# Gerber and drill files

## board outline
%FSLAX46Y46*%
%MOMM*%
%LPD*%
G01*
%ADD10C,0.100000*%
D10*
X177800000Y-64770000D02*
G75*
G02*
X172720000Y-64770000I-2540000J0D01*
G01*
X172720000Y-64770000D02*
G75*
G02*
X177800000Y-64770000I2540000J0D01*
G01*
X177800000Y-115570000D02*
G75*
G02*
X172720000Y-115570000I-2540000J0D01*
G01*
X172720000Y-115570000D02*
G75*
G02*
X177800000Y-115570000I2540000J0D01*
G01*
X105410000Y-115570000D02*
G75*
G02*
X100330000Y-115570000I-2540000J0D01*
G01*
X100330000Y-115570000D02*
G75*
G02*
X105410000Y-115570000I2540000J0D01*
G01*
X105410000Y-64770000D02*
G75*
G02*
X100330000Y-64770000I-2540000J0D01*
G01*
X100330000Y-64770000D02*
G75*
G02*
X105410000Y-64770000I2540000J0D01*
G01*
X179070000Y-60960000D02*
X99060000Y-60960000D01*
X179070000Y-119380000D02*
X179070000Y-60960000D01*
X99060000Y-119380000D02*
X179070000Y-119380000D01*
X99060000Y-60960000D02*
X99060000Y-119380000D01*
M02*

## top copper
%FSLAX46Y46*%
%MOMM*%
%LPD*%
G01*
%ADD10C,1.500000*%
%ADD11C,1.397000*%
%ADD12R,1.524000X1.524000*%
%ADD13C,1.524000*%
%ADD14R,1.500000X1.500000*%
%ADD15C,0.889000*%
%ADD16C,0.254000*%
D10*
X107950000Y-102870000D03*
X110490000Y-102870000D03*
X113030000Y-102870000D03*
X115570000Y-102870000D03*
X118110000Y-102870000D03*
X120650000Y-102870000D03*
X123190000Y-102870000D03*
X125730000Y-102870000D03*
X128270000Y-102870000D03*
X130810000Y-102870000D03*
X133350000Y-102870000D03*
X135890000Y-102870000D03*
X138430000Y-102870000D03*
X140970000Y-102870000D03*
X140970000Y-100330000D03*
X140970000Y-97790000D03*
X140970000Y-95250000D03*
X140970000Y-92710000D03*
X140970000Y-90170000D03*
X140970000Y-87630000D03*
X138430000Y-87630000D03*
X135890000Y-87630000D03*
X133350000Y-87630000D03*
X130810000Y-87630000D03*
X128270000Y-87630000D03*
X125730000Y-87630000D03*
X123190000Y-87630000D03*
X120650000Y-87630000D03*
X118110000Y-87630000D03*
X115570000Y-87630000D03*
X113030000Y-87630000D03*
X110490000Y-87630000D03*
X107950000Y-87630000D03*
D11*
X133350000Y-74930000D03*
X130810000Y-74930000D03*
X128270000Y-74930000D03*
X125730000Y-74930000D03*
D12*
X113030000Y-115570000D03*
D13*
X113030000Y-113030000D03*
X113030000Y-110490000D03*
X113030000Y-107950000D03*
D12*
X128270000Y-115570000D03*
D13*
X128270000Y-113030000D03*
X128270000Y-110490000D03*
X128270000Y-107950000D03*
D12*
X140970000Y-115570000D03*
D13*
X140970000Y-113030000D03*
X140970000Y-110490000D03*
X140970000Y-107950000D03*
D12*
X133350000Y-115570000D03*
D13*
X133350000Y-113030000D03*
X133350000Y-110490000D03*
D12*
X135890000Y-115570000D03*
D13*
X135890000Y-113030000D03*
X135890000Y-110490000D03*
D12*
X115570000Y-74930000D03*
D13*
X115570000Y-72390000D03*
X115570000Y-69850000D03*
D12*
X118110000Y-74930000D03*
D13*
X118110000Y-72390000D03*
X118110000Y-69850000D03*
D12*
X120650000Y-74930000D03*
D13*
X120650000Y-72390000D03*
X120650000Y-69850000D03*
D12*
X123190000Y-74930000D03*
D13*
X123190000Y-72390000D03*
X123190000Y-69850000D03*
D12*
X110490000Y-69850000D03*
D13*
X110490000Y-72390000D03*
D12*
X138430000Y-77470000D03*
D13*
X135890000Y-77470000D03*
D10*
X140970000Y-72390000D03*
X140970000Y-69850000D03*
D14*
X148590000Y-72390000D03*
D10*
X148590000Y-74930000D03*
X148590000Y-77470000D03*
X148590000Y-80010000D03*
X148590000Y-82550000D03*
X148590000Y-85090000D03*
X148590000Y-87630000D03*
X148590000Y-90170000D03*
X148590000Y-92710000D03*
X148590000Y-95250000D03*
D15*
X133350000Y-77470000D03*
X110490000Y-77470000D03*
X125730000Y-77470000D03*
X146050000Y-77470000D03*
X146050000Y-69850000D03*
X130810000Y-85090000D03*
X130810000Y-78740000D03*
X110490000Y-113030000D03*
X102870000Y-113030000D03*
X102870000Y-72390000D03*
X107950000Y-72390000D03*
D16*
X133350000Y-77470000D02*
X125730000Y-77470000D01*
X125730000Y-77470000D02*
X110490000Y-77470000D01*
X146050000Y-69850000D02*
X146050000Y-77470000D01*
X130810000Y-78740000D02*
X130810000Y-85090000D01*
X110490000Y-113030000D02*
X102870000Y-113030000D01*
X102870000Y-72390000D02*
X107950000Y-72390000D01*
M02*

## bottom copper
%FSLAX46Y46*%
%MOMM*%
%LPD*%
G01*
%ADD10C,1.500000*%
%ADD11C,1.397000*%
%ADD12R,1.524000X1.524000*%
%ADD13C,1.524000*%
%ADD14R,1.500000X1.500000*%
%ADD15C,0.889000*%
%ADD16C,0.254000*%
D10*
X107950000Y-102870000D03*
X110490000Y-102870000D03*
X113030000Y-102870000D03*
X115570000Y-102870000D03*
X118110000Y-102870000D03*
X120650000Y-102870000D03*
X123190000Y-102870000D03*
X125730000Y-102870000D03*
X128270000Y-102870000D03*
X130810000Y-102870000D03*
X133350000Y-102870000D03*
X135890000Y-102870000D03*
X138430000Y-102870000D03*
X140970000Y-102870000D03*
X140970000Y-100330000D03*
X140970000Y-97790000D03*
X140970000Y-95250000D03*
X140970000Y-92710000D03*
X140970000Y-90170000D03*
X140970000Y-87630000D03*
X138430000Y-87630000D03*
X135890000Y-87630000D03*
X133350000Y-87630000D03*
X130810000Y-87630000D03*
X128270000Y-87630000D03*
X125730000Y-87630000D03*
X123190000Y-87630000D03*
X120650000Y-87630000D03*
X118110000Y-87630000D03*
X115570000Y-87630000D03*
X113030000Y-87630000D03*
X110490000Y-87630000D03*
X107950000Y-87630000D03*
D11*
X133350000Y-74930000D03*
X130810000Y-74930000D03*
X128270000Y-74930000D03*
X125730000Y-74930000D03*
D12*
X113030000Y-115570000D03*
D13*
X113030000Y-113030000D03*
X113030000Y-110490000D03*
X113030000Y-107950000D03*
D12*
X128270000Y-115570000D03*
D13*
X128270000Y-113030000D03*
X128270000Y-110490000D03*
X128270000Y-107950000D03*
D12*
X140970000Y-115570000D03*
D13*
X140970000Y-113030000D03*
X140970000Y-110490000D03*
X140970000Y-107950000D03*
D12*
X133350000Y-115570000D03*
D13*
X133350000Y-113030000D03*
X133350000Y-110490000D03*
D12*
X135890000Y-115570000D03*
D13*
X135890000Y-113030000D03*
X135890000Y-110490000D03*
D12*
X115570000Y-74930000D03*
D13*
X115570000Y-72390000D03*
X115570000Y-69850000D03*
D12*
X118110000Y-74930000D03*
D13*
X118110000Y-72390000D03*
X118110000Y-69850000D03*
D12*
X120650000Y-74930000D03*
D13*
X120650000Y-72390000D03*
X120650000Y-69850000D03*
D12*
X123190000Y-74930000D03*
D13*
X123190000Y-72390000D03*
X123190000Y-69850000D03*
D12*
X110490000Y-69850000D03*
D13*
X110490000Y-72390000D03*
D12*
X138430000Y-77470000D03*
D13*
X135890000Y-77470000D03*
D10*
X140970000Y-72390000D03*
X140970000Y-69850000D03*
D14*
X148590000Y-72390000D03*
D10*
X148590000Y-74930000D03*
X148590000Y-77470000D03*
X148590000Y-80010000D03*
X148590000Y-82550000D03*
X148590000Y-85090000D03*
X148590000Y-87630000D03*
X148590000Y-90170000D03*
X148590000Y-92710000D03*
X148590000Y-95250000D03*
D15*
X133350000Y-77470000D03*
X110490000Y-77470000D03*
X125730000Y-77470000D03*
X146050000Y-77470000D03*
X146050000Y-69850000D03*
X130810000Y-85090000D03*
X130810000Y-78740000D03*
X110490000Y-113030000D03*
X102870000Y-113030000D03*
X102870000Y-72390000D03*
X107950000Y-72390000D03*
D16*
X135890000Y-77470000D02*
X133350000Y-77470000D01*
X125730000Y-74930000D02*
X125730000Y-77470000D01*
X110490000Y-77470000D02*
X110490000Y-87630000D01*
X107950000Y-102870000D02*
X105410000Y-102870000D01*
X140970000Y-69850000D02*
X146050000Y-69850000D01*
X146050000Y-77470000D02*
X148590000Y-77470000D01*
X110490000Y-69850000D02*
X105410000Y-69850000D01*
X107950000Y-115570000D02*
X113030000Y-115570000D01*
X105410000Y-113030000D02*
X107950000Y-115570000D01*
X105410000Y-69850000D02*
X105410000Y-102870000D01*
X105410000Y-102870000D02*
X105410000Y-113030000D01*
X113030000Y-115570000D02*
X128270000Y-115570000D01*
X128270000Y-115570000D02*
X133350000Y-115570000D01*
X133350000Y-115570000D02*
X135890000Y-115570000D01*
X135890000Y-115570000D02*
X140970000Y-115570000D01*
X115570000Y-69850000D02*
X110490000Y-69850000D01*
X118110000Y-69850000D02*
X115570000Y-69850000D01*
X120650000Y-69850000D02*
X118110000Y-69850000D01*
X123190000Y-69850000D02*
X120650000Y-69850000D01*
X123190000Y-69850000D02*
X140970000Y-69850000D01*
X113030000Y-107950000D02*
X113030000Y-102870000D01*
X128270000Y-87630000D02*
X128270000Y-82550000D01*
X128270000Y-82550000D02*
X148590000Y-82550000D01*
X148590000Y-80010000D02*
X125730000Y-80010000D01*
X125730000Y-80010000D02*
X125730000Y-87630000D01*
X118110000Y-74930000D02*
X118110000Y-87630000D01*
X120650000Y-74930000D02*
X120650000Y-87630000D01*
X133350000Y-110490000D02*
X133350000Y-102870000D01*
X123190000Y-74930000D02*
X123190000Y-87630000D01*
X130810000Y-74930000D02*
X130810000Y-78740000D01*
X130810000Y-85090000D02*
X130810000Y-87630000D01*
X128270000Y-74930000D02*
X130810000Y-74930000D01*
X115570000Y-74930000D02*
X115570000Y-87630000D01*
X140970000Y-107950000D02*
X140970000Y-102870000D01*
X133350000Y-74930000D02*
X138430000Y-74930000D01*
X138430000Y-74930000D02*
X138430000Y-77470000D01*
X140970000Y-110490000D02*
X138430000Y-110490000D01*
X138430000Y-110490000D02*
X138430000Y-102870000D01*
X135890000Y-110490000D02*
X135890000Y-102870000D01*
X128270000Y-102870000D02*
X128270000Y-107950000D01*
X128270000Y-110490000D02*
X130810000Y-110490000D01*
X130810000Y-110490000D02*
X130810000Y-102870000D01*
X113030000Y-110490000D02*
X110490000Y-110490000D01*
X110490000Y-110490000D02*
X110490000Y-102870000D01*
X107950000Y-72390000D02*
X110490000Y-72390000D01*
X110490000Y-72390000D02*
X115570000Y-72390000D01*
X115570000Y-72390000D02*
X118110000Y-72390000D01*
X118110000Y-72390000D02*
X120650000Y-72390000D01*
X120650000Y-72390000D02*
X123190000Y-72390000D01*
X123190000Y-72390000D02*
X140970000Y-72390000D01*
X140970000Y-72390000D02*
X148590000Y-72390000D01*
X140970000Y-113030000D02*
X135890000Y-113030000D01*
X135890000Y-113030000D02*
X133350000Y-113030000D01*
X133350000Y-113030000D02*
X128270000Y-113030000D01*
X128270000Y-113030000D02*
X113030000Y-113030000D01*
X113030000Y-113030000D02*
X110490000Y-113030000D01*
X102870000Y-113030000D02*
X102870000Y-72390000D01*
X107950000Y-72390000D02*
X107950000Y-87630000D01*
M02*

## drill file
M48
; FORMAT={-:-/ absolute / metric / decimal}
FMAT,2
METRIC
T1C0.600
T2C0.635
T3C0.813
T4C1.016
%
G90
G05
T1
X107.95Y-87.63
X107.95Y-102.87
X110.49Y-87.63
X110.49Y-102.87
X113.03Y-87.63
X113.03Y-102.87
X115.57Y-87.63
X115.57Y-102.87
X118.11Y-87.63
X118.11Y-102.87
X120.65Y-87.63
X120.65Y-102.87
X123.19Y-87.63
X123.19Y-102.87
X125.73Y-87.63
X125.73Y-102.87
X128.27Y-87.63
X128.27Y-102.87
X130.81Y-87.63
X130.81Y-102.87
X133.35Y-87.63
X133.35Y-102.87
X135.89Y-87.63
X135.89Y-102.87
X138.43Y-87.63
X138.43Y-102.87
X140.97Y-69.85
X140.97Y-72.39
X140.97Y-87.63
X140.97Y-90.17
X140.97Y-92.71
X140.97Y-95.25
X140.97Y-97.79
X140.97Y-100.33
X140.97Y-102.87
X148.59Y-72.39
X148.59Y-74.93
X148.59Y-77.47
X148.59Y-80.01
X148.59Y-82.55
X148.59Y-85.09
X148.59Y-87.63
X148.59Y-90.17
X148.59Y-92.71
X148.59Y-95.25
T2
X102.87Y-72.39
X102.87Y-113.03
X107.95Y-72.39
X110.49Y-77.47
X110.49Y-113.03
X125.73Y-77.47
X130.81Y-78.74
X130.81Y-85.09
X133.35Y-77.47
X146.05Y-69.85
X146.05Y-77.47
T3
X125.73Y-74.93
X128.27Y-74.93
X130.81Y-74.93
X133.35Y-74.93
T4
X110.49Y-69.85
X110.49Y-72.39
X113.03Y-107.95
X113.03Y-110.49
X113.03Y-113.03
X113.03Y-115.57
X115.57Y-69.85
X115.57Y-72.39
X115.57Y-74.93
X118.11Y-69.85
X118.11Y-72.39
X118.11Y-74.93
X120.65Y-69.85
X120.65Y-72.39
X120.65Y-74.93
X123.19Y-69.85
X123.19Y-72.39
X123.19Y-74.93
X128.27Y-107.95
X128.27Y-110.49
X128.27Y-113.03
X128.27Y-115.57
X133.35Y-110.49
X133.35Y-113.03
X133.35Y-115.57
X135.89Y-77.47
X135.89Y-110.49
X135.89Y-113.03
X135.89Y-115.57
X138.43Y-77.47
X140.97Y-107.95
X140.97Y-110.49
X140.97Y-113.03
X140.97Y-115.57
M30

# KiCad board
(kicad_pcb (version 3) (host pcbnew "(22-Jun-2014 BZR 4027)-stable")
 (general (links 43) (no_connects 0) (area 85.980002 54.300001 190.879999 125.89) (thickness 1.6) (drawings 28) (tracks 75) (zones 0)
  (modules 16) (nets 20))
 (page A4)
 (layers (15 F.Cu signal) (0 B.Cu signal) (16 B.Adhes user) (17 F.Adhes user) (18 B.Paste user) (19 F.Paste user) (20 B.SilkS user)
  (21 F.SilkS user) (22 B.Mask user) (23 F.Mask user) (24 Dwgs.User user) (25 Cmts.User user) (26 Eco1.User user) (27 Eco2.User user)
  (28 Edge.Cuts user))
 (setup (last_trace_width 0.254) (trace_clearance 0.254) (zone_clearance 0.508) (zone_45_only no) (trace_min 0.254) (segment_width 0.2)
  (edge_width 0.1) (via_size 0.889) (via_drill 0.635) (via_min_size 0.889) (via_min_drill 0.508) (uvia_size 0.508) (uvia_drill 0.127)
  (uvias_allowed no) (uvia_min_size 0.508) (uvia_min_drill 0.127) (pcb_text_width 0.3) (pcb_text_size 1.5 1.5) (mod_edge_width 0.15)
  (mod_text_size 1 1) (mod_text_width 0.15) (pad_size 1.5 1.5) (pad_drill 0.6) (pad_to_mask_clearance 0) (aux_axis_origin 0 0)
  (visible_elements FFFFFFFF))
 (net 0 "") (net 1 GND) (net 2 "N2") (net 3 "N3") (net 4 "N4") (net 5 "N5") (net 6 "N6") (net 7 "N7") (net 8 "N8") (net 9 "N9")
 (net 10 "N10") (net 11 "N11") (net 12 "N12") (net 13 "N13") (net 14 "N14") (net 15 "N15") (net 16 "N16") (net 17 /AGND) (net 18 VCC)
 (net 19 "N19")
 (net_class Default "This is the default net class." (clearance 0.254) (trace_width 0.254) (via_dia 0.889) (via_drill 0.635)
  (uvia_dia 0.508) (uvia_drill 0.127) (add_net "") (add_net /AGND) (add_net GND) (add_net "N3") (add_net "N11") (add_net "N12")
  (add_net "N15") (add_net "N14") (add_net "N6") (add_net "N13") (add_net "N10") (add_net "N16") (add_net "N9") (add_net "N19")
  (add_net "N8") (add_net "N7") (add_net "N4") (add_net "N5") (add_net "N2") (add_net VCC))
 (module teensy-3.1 (layer F.Cu) (at 124.46 95.25 90)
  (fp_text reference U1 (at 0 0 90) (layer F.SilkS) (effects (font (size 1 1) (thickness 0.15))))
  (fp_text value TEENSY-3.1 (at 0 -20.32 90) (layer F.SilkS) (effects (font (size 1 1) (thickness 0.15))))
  (pad 1 thru_hole circle (at -7.62 -16.51 90) (size 1.5 1.5) (drill 0.6) (layers *.Cu *.Mask F.SilkS) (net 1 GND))
  (pad 2 thru_hole circle (at -7.62 -13.97 90) (size 1.5 1.5) (drill 0.6) (layers *.Cu *.Mask F.SilkS) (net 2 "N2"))
  (pad 3 thru_hole circle (at -7.62 -11.43 90) (size 1.5 1.5) (drill 0.6) (layers *.Cu *.Mask F.SilkS) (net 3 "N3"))
  (pad 4 thru_hole circle (at -7.62 -8.89 90) (size 1.5 1.5) (drill 0.6) (layers *.Cu *.Mask F.SilkS))
  (pad 5 thru_hole circle (at -7.62 -6.35 90) (size 1.5 1.5) (drill 0.6) (layers *.Cu *.Mask F.SilkS))
  (pad 6 thru_hole circle (at -7.62 -3.81 90) (size 1.5 1.5) (drill 0.6) (layers *.Cu *.Mask F.SilkS))
  (pad 7 thru_hole circle (at -7.62 -1.27 90) (size 1.5 1.5) (drill 0.6) (layers *.Cu *.Mask F.SilkS))
  (pad 8 thru_hole circle (at -7.62 1.27 90) (size 1.5 1.5) (drill 0.6) (layers *.Cu *.Mask F.SilkS))
  (pad 9 thru_hole circle (at -7.62 3.81 90) (size 1.5 1.5) (drill 0.6) (layers *.Cu *.Mask F.SilkS) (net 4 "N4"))
  (pad 10 thru_hole circle (at -7.62 6.35 90) (size 1.5 1.5) (drill 0.6) (layers *.Cu *.Mask F.SilkS) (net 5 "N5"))
  (pad 11 thru_hole circle (at -7.62 8.89 90) (size 1.5 1.5) (drill 0.6) (layers *.Cu *.Mask F.SilkS) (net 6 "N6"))
  (pad 12 thru_hole circle (at -7.62 11.43 90) (size 1.5 1.5) (drill 0.6) (layers *.Cu *.Mask F.SilkS) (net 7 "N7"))
  (pad 13 thru_hole circle (at -7.62 13.97 90) (size 1.5 1.5) (drill 0.6) (layers *.Cu *.Mask F.SilkS) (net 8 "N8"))
  (pad 14 thru_hole circle (at -7.62 16.51 90) (size 1.5 1.5) (drill 0.6) (layers *.Cu *.Mask F.SilkS) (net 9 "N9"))
  (pad 15 thru_hole circle (at -5.08 16.51 90) (size 1.5 1.5) (drill 0.6) (layers *.Cu *.Mask F.SilkS))
  (pad 16 thru_hole circle (at -2.54 16.51 90) (size 1.5 1.5) (drill 0.6) (layers *.Cu *.Mask F.SilkS))
  (pad 17 thru_hole circle (at 0 16.51 90) (size 1.5 1.5) (drill 0.6) (layers *.Cu *.Mask F.SilkS))
  (pad 18 thru_hole circle (at 2.54 16.51 90) (size 1.5 1.5) (drill 0.6) (layers *.Cu *.Mask F.SilkS))
  (pad 19 thru_hole circle (at 5.08 16.51 90) (size 1.5 1.5) (drill 0.6) (layers *.Cu *.Mask F.SilkS))
  (pad 20 thru_hole circle (at 7.62 16.51 90) (size 1.5 1.5) (drill 0.6) (layers *.Cu *.Mask F.SilkS))
  (pad 21 thru_hole circle (at 7.62 13.97 90) (size 1.5 1.5) (drill 0.6) (layers *.Cu *.Mask F.SilkS))
  (pad 22 thru_hole circle (at 7.62 11.43 90) (size 1.5 1.5) (drill 0.6) (layers *.Cu *.Mask F.SilkS))
  (pad 23 thru_hole circle (at 7.62 8.89 90) (size 1.5 1.5) (drill 0.6) (layers *.Cu *.Mask F.SilkS))
  (pad 24 thru_hole circle (at 7.62 6.35 90) (size 1.5 1.5) (drill 0.6) (layers *.Cu *.Mask F.SilkS) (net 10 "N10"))
  (pad 25 thru_hole circle (at 7.62 3.81 90) (size 1.5 1.5) (drill 0.6) (layers *.Cu *.Mask F.SilkS) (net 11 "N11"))
  (pad 26 thru_hole circle (at 7.62 1.27 90) (size 1.5 1.5) (drill 0.6) (layers *.Cu *.Mask F.SilkS) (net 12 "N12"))
  (pad 27 thru_hole circle (at 7.62 -1.27 90) (size 1.5 1.5) (drill 0.6) (layers *.Cu *.Mask F.SilkS) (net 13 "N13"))
  (pad 28 thru_hole circle (at 7.62 -3.81 90) (size 1.5 1.5) (drill 0.6) (layers *.Cu *.Mask F.SilkS) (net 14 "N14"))
  (pad 29 thru_hole circle (at 7.62 -6.35 90) (size 1.5 1.5) (drill 0.6) (layers *.Cu *.Mask F.SilkS) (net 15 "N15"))
  (pad 30 thru_hole circle (at 7.62 -8.89 90) (size 1.5 1.5) (drill 0.6) (layers *.Cu *.Mask F.SilkS) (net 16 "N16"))
  (pad 31 thru_hole circle (at 7.62 -11.43 90) (size 1.5 1.5) (drill 0.6) (layers *.Cu *.Mask F.SilkS))
  (pad 32 thru_hole circle (at 7.62 -13.97 90) (size 1.5 1.5) (drill 0.6) (layers *.Cu *.Mask F.SilkS) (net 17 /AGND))
  (pad 33 thru_hole circle (at 7.62 -16.51 90) (size 1.5 1.5) (drill 0.6) (layers *.Cu *.Mask F.SilkS) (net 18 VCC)))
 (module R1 (layer F.Cu) (at 132.08 74.93 180) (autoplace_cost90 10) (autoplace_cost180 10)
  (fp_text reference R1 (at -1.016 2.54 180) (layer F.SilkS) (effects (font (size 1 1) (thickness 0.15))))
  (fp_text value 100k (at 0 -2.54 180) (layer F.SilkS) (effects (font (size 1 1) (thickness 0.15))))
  (pad 1 thru_hole circle (at -1.27 0 180) (size 1.397 1.397) (drill 0.8128) (layers *.Cu *.Mask F.SilkS) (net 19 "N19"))
  (pad 2 thru_hole circle (at 1.27 0 180) (size 1.397 1.397) (drill 0.8128) (layers *.Cu *.Mask F.SilkS) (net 10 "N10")))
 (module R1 (layer F.Cu) (at 127 74.93 180) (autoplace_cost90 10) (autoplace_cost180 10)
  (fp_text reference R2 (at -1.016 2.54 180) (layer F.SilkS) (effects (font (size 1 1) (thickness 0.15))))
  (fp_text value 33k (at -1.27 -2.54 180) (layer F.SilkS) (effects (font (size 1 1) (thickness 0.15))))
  (pad 1 thru_hole circle (at -1.27 0 180) (size 1.397 1.397) (drill 0.8128) (layers *.Cu *.Mask F.SilkS) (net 10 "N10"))
  (pad 2 thru_hole circle (at 1.27 0 180) (size 1.397 1.397) (drill 0.8128) (layers *.Cu *.Mask F.SilkS) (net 17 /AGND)))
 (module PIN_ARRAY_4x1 (layer F.Cu) (at 113.03 111.76 90)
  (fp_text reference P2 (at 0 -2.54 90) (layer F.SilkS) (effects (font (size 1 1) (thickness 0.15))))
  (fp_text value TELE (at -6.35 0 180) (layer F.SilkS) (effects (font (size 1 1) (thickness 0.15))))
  (pad 1 thru_hole rect (at -3.81 0 90) (size 1.524 1.524) (drill 1.016) (layers *.Cu *.Mask F.SilkS) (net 1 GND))
  (pad 2 thru_hole circle (at -1.27 0 90) (size 1.524 1.524) (drill 1.016) (layers *.Cu *.Mask F.SilkS) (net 18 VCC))
  (pad 3 thru_hole circle (at 1.27 0 90) (size 1.524 1.524) (drill 1.016) (layers *.Cu *.Mask F.SilkS) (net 2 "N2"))
  (pad 4 thru_hole circle (at 3.81 0 90) (size 1.524 1.524) (drill 1.016) (layers *.Cu *.Mask F.SilkS) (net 3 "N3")))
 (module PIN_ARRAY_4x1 (layer F.Cu) (at 128.27 111.76 90)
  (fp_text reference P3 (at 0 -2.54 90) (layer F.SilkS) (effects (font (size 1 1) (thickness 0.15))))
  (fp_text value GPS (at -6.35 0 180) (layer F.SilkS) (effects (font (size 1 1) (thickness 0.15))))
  (pad 1 thru_hole rect (at -3.81 0 90) (size 1.524 1.524) (drill 1.016) (layers *.Cu *.Mask F.SilkS) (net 1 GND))
  (pad 2 thru_hole circle (at -1.27 0 90) (size 1.524 1.524) (drill 1.016) (layers *.Cu *.Mask F.SilkS) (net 18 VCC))
  (pad 3 thru_hole circle (at 1.27 0 90) (size 1.524 1.524) (drill 1.016) (layers *.Cu *.Mask F.SilkS) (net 5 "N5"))
  (pad 4 thru_hole circle (at 3.81 0 90) (size 1.524 1.524) (drill 1.016) (layers *.Cu *.Mask F.SilkS) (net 4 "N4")))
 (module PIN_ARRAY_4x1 (layer F.Cu) (at 140.97 111.76 90)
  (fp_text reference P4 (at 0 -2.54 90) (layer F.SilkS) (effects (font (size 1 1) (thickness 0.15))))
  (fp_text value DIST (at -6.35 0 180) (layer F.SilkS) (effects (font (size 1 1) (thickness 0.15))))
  (pad 1 thru_hole rect (at -3.81 0 90) (size 1.524 1.524) (drill 1.016) (layers *.Cu *.Mask F.SilkS) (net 1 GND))
  (pad 2 thru_hole circle (at -1.27 0 90) (size 1.524 1.524) (drill 1.016) (layers *.Cu *.Mask F.SilkS) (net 18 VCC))
  (pad 3 thru_hole circle (at 1.27 0 90) (size 1.524 1.524) (drill 1.016) (layers *.Cu *.Mask F.SilkS) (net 8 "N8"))
  (pad 4 thru_hole circle (at 3.81 0 90) (size 1.524 1.524) (drill 1.016) (layers *.Cu *.Mask F.SilkS) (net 9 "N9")))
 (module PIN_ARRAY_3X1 (layer F.Cu) (at 133.35 113.03 90)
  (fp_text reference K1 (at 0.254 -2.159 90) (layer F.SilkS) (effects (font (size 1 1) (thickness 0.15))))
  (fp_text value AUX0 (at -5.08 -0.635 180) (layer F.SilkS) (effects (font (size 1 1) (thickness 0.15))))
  (pad 1 thru_hole rect (at -2.54 0 90) (size 1.524 1.524) (drill 1.016) (layers *.Cu *.Mask F.SilkS) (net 1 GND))
  (pad 2 thru_hole circle (at 0 0 90) (size 1.524 1.524) (drill 1.016) (layers *.Cu *.Mask F.SilkS) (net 18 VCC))
  (pad 3 thru_hole circle (at 2.54 0 90) (size 1.524 1.524) (drill 1.016) (layers *.Cu *.Mask F.SilkS) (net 6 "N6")))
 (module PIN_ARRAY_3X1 (layer F.Cu) (at 135.89 113.03 90)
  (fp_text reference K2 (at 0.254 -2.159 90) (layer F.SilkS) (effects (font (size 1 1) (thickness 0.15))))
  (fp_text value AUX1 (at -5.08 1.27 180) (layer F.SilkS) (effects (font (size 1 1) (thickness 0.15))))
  (pad 1 thru_hole rect (at -2.54 0 90) (size 1.524 1.524) (drill 1.016) (layers *.Cu *.Mask F.SilkS) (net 1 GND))
  (pad 2 thru_hole circle (at 0 0 90) (size 1.524 1.524) (drill 1.016) (layers *.Cu *.Mask F.SilkS) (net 18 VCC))
  (pad 3 thru_hole circle (at 2.54 0 90) (size 1.524 1.524) (drill 1.016) (layers *.Cu *.Mask F.SilkS) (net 7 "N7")))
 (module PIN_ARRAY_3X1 (layer F.Cu) (at 115.57 72.39 90)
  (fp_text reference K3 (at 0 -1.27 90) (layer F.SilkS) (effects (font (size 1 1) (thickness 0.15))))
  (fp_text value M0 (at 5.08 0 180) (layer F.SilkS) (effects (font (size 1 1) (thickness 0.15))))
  (pad 1 thru_hole rect (at -2.54 0 90) (size 1.524 1.524) (drill 1.016) (layers *.Cu *.Mask F.SilkS) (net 16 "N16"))
  (pad 2 thru_hole circle (at 0 0 90) (size 1.524 1.524) (drill 1.016) (layers *.Cu *.Mask F.SilkS) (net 18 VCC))
  (pad 3 thru_hole circle (at 2.54 0 90) (size 1.524 1.524) (drill 1.016) (layers *.Cu *.Mask F.SilkS) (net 1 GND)))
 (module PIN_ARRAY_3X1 (layer F.Cu) (at 118.11 72.39 90)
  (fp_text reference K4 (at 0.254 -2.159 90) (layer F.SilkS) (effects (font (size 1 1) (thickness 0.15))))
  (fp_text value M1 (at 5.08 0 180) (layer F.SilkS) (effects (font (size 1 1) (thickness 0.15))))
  (pad 1 thru_hole rect (at -2.54 0 90) (size 1.524 1.524) (drill 1.016) (layers *.Cu *.Mask F.SilkS) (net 15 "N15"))
  (pad 2 thru_hole circle (at 0 0 90) (size 1.524 1.524) (drill 1.016) (layers *.Cu *.Mask F.SilkS) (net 18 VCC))
  (pad 3 thru_hole circle (at 2.54 0 90) (size 1.524 1.524) (drill 1.016) (layers *.Cu *.Mask F.SilkS) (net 1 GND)))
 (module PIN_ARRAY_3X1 (layer F.Cu) (at 120.65 72.39 90)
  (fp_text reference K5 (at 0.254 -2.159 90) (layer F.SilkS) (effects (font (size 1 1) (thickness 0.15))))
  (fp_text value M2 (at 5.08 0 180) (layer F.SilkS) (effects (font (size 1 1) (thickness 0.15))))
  (pad 1 thru_hole rect (at -2.54 0 90) (size 1.524 1.524) (drill 1.016) (layers *.Cu *.Mask F.SilkS) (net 14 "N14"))
  (pad 2 thru_hole circle (at 0 0 90) (size 1.524 1.524) (drill 1.016) (layers *.Cu *.Mask F.SilkS) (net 18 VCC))
  (pad 3 thru_hole circle (at 2.54 0 90) (size 1.524 1.524) (drill 1.016) (layers *.Cu *.Mask F.SilkS) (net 1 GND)))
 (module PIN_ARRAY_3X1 (layer F.Cu) (at 123.19 72.39 90)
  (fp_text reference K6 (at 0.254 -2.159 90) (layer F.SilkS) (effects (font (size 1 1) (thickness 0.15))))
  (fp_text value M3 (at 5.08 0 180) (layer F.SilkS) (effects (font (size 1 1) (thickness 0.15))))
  (pad 1 thru_hole rect (at -2.54 0 90) (size 1.524 1.524) (drill 1.016) (layers *.Cu *.Mask F.SilkS) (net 13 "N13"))
  (pad 2 thru_hole circle (at 0 0 90) (size 1.524 1.524) (drill 1.016) (layers *.Cu *.Mask F.SilkS) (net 18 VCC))
  (pad 3 thru_hole circle (at 2.54 0 90) (size 1.524 1.524) (drill 1.016) (layers *.Cu *.Mask F.SilkS) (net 1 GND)))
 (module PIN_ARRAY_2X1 (layer F.Cu) (at 110.49 71.12 270)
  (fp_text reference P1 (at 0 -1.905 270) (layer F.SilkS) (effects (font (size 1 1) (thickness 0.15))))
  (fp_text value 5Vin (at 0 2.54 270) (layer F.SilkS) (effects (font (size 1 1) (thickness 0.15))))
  (pad 1 thru_hole rect (at -1.27 0 270) (size 1.524 1.524) (drill 1.016) (layers *.Cu *.Mask F.SilkS) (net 1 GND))
  (pad 2 thru_hole circle (at 1.27 0 270) (size 1.524 1.524) (drill 1.016) (layers *.Cu *.Mask F.SilkS) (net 18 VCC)))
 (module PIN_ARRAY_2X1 (layer F.Cu) (at 137.16 77.47 180)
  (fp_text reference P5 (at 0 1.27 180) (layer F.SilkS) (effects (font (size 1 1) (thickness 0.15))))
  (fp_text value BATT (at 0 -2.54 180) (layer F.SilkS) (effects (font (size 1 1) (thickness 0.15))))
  (pad 1 thru_hole rect (at -1.27 0 180) (size 1.524 1.524) (drill 1.016) (layers *.Cu *.Mask F.SilkS) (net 19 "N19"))
  (pad 2 thru_hole circle (at 1.27 0 180) (size 1.524 1.524) (drill 1.016) (layers *.Cu *.Mask F.SilkS) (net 17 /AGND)))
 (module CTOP (layer F.Cu) (at 140.97 71.12 90)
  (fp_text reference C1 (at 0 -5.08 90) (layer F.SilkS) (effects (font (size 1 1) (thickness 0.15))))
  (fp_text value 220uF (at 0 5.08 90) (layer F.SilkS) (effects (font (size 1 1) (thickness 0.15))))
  (pad 1 thru_hole circle (at -1.27 0 90) (size 1.5 1.5) (drill 0.6) (layers *.Cu *.Mask F.SilkS) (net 18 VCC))
  (pad 2 thru_hole circle (at 1.27 0 90) (size 1.5 1.5) (drill 0.6) (layers *.Cu *.Mask F.SilkS) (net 1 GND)))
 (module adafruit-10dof (layer F.Cu) (at 157.48 83.82 270)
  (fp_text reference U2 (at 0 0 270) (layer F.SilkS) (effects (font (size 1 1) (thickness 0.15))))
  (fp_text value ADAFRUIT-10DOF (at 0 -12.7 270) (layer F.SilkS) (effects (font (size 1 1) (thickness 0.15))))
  (pad 1 thru_hole rect (at -11.43 8.89 270) (size 1.5 1.5) (drill 0.6) (layers *.Cu *.Mask F.SilkS) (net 18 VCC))
  (pad 2 thru_hole circle (at -8.89 8.89 270) (size 1.5 1.5) (drill 0.6) (layers *.Cu *.Mask F.SilkS))
  (pad 3 thru_hole circle (at -6.35 8.89 270) (size 1.5 1.5) (drill 0.6) (layers *.Cu *.Mask F.SilkS) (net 1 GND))
  (pad 4 thru_hole circle (at -3.81 8.89 270) (size 1.5 1.5) (drill 0.6) (layers *.Cu *.Mask F.SilkS) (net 12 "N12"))
  (pad 5 thru_hole circle (at -1.27 8.89 270) (size 1.5 1.5) (drill 0.6) (layers *.Cu *.Mask F.SilkS) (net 11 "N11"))
  (pad 6 thru_hole circle (at 1.27 8.89 270) (size 1.5 1.5) (drill 0.6) (layers *.Cu *.Mask F.SilkS))
  (pad 7 thru_hole circle (at 3.81 8.89 270) (size 1.5 1.5) (drill 0.6) (layers *.Cu *.Mask F.SilkS))
  (pad 8 thru_hole circle (at 6.35 8.89 270) (size 1.5 1.5) (drill 0.6) (layers *.Cu *.Mask F.SilkS))
  (pad 9 thru_hole circle (at 8.89 8.89 270) (size 1.5 1.5) (drill 0.6) (layers *.Cu *.Mask F.SilkS))
  (pad 10 thru_hole circle (at 11.43 8.89 270) (size 1.5 1.5) (drill 0.6) (layers *.Cu *.Mask F.SilkS)))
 (gr_circle (center 175.26 64.77) (end 177.8 64.77) (layer Edge.Cuts) (width 0.1))
 (gr_circle (center 175.26 115.57) (end 177.8 115.57) (layer Edge.Cuts) (width 0.1))
 (gr_circle (center 102.87 115.57) (end 105.41 115.57) (layer Edge.Cuts) (width 0.1))
 (gr_circle (center 102.87 64.77) (end 105.41 64.77) (layer Edge.Cuts) (width 0.1))
 (gr_line (start 179.07 60.96) (end 99.06 60.96) (angle 90) (layer Edge.Cuts) (width 0.1))
 (gr_line (start 179.07 119.38) (end 179.07 60.96) (angle 90) (layer Edge.Cuts) (width 0.1))
 (gr_line (start 99.06 119.38) (end 179.07 119.38) (angle 90) (layer Edge.Cuts) (width 0.1))
 (gr_line (start 99.06 60.96) (end 99.06 119.38) (angle 90) (layer Edge.Cuts) (width 0.1))
 (segment (start 135.89 77.47) (end 133.35 77.47) (width 0.254) (layer B.Cu) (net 17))
 (segment (start 133.35 77.47) (end 125.73 77.47) (width 0.254) (layer F.Cu) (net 17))
 (via (at 133.35 77.47) (size 0.889) (layers F.Cu B.Cu) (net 17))
 (segment (start 125.73 74.93) (end 125.73 77.47) (width 0.254) (layer B.Cu) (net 17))
 (segment (start 110.49 77.47) (end 110.49 87.63) (width 0.254) (layer B.Cu) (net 17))
 (via (at 110.49 77.47) (size 0.889) (layers F.Cu B.Cu) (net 17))
 (segment (start 125.73 77.47) (end 110.49 77.47) (width 0.254) (layer F.Cu) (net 17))
 (via (at 125.73 77.47) (size 0.889) (layers F.Cu B.Cu) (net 17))
 (segment (start 107.95 102.87) (end 105.41 102.87) (width 0.254) (layer B.Cu) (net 1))
 (segment (start 140.97 69.85) (end 146.05 69.85) (width 0.254) (layer B.Cu) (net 1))
 (segment (start 146.05 77.47) (end 148.59 77.47) (width 0.254) (layer B.Cu) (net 1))
 (via (at 146.05 77.47) (size 0.889) (layers F.Cu B.Cu) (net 1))
 (segment (start 146.05 69.85) (end 146.05 77.47) (width 0.254) (layer F.Cu) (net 1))
 (via (at 146.05 69.85) (size 0.889) (layers F.Cu B.Cu) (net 1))
 (segment (start 110.49 69.85) (end 105.41 69.85) (width 0.254) (layer B.Cu) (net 1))
 (segment (start 107.95 115.57) (end 113.03 115.57) (width 0.254) (layer B.Cu) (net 1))
 (segment (start 105.41 113.03) (end 107.95 115.57) (width 0.254) (layer B.Cu) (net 1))
 (segment (start 105.41 69.85) (end 105.41 102.87) (width 0.254) (layer B.Cu) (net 1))
 (segment (start 105.41 102.87) (end 105.41 113.03) (width 0.254) (layer B.Cu) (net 1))
 (segment (start 113.03 115.57) (end 128.27 115.57) (width 0.254) (layer B.Cu) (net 1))
 (segment (start 128.27 115.57) (end 133.35 115.57) (width 0.254) (layer B.Cu) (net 1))
 (segment (start 133.35 115.57) (end 135.89 115.57) (width 0.254) (layer B.Cu) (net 1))
 (segment (start 135.89 115.57) (end 140.97 115.57) (width 0.254) (layer B.Cu) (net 1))
 (segment (start 115.57 69.85) (end 110.49 69.85) (width 0.254) (layer B.Cu) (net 1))
 (segment (start 118.11 69.85) (end 115.57 69.85) (width 0.254) (layer B.Cu) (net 1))
 (segment (start 120.65 69.85) (end 118.11 69.85) (width 0.254) (layer B.Cu) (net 1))
 (segment (start 123.19 69.85) (end 120.65 69.85) (width 0.254) (layer B.Cu) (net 1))
 (segment (start 123.19 69.85) (end 140.97 69.85) (width 0.254) (layer B.Cu) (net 1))
 (segment (start 113.03 107.95) (end 113.03 102.87) (width 0.254) (layer B.Cu) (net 3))
 (segment (start 128.27 87.63) (end 128.27 82.55) (width 0.254) (layer B.Cu) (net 11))
 (segment (start 128.27 82.55) (end 148.59 82.55) (width 0.254) (layer B.Cu) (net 11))
 (segment (start 148.59 80.01) (end 125.73 80.01) (width 0.254) (layer B.Cu) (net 12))
 (segment (start 125.73 80.01) (end 125.73 87.63) (width 0.254) (layer B.Cu) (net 12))
 (segment (start 118.11 74.93) (end 118.11 87.63) (width 0.254) (layer B.Cu) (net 15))
 (segment (start 120.65 74.93) (end 120.65 87.63) (width 0.254) (layer B.Cu) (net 14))
 (segment (start 133.35 110.49) (end 133.35 102.87) (width 0.254) (layer B.Cu) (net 6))
 (segment (start 123.19 74.93) (end 123.19 87.63) (width 0.254) (layer B.Cu) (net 13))
 (segment (start 130.81 74.93) (end 130.81 78.74) (width 0.254) (layer B.Cu) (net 10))
 (segment (start 130.81 85.09) (end 130.81 87.63) (width 0.254) (layer B.Cu) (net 10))
 (via (at 130.81 85.09) (size 0.889) (layers F.Cu B.Cu) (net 10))
 (segment (start 130.81 78.74) (end 130.81 85.09) (width 0.254) (layer F.Cu) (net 10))
 (via (at 130.81 78.74) (size 0.889) (layers F.Cu B.Cu) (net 10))
 (segment (start 128.27 74.93) (end 130.81 74.93) (width 0.254) (layer B.Cu) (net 10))
 (segment (start 115.57 74.93) (end 115.57 87.63) (width 0.254) (layer B.Cu) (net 16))
 (segment (start 140.97 107.95) (end 140.97 102.87) (width 0.254) (layer B.Cu) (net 9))
 (segment (start 133.35 74.93) (end 138.43 74.93) (width 0.254) (layer B.Cu) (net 19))
 (segment (start 138.43 74.93) (end 138.43 77.47) (width 0.254) (layer B.Cu) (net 19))
 (segment (start 140.97 110.49) (end 138.43 110.49) (width 0.254) (layer B.Cu) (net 8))
 (segment (start 138.43 110.49) (end 138.43 102.87) (width 0.254) (layer B.Cu) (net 8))
 (segment (start 135.89 110.49) (end 135.89 102.87) (width 0.254) (layer B.Cu) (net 7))
 (segment (start 128.27 102.87) (end 128.27 107.95) (width 0.254) (layer B.Cu) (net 4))
 (segment (start 128.27 110.49) (end 130.81 110.49) (width 0.254) (layer B.Cu) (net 5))
 (segment (start 130.81 110.49) (end 130.81 102.87) (width 0.254) (layer B.Cu) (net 5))
 (segment (start 113.03 110.49) (end 110.49 110.49) (width 0.254) (layer B.Cu) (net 2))
 (segment (start 110.49 110.49) (end 110.49 102.87) (width 0.254) (layer B.Cu) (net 2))
 (segment (start 107.95 72.39) (end 110.49 72.39) (width 0.254) (layer B.Cu) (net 18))
 (segment (start 110.49 72.39) (end 115.57 72.39) (width 0.254) (layer B.Cu) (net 18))
 (segment (start 115.57 72.39) (end 118.11 72.39) (width 0.254) (layer B.Cu) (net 18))
 (segment (start 118.11 72.39) (end 120.65 72.39) (width 0.254) (layer B.Cu) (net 18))
 (segment (start 120.65 72.39) (end 123.19 72.39) (width 0.254) (layer B.Cu) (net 18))
 (segment (start 123.19 72.39) (end 140.97 72.39) (width 0.254) (layer B.Cu) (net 18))
 (segment (start 140.97 72.39) (end 148.59 72.39) (width 0.254) (layer B.Cu) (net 18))
 (segment (start 140.97 113.03) (end 135.89 113.03) (width 0.254) (layer B.Cu) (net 18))
 (segment (start 135.89 113.03) (end 133.35 113.03) (width 0.254) (layer B.Cu) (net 18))
 (segment (start 133.35 113.03) (end 128.27 113.03) (width 0.254) (layer B.Cu) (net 18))
 (segment (start 128.27 113.03) (end 113.03 113.03) (width 0.254) (layer B.Cu) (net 18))
 (segment (start 113.03 113.03) (end 110.49 113.03) (width 0.254) (layer B.Cu) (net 18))
 (via (at 110.49 113.03) (size 0.889) (layers F.Cu B.Cu) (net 18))
 (segment (start 110.49 113.03) (end 102.87 113.03) (width 0.254) (layer F.Cu) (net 18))
 (via (at 102.87 113.03) (size 0.889) (layers F.Cu B.Cu) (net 18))
 (segment (start 102.87 113.03) (end 102.87 72.39) (width 0.254) (layer B.Cu) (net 18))
 (via (at 102.87 72.39) (size 0.889) (layers F.Cu B.Cu) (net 18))
 (segment (start 102.87 72.39) (end 107.95 72.39) (width 0.254) (layer F.Cu) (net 18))
 (via (at 107.95 72.39) (size 0.889) (layers F.Cu B.Cu) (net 18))
 (segment (start 107.95 72.39) (end 107.95 87.63) (width 0.254) (layer B.Cu) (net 18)))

